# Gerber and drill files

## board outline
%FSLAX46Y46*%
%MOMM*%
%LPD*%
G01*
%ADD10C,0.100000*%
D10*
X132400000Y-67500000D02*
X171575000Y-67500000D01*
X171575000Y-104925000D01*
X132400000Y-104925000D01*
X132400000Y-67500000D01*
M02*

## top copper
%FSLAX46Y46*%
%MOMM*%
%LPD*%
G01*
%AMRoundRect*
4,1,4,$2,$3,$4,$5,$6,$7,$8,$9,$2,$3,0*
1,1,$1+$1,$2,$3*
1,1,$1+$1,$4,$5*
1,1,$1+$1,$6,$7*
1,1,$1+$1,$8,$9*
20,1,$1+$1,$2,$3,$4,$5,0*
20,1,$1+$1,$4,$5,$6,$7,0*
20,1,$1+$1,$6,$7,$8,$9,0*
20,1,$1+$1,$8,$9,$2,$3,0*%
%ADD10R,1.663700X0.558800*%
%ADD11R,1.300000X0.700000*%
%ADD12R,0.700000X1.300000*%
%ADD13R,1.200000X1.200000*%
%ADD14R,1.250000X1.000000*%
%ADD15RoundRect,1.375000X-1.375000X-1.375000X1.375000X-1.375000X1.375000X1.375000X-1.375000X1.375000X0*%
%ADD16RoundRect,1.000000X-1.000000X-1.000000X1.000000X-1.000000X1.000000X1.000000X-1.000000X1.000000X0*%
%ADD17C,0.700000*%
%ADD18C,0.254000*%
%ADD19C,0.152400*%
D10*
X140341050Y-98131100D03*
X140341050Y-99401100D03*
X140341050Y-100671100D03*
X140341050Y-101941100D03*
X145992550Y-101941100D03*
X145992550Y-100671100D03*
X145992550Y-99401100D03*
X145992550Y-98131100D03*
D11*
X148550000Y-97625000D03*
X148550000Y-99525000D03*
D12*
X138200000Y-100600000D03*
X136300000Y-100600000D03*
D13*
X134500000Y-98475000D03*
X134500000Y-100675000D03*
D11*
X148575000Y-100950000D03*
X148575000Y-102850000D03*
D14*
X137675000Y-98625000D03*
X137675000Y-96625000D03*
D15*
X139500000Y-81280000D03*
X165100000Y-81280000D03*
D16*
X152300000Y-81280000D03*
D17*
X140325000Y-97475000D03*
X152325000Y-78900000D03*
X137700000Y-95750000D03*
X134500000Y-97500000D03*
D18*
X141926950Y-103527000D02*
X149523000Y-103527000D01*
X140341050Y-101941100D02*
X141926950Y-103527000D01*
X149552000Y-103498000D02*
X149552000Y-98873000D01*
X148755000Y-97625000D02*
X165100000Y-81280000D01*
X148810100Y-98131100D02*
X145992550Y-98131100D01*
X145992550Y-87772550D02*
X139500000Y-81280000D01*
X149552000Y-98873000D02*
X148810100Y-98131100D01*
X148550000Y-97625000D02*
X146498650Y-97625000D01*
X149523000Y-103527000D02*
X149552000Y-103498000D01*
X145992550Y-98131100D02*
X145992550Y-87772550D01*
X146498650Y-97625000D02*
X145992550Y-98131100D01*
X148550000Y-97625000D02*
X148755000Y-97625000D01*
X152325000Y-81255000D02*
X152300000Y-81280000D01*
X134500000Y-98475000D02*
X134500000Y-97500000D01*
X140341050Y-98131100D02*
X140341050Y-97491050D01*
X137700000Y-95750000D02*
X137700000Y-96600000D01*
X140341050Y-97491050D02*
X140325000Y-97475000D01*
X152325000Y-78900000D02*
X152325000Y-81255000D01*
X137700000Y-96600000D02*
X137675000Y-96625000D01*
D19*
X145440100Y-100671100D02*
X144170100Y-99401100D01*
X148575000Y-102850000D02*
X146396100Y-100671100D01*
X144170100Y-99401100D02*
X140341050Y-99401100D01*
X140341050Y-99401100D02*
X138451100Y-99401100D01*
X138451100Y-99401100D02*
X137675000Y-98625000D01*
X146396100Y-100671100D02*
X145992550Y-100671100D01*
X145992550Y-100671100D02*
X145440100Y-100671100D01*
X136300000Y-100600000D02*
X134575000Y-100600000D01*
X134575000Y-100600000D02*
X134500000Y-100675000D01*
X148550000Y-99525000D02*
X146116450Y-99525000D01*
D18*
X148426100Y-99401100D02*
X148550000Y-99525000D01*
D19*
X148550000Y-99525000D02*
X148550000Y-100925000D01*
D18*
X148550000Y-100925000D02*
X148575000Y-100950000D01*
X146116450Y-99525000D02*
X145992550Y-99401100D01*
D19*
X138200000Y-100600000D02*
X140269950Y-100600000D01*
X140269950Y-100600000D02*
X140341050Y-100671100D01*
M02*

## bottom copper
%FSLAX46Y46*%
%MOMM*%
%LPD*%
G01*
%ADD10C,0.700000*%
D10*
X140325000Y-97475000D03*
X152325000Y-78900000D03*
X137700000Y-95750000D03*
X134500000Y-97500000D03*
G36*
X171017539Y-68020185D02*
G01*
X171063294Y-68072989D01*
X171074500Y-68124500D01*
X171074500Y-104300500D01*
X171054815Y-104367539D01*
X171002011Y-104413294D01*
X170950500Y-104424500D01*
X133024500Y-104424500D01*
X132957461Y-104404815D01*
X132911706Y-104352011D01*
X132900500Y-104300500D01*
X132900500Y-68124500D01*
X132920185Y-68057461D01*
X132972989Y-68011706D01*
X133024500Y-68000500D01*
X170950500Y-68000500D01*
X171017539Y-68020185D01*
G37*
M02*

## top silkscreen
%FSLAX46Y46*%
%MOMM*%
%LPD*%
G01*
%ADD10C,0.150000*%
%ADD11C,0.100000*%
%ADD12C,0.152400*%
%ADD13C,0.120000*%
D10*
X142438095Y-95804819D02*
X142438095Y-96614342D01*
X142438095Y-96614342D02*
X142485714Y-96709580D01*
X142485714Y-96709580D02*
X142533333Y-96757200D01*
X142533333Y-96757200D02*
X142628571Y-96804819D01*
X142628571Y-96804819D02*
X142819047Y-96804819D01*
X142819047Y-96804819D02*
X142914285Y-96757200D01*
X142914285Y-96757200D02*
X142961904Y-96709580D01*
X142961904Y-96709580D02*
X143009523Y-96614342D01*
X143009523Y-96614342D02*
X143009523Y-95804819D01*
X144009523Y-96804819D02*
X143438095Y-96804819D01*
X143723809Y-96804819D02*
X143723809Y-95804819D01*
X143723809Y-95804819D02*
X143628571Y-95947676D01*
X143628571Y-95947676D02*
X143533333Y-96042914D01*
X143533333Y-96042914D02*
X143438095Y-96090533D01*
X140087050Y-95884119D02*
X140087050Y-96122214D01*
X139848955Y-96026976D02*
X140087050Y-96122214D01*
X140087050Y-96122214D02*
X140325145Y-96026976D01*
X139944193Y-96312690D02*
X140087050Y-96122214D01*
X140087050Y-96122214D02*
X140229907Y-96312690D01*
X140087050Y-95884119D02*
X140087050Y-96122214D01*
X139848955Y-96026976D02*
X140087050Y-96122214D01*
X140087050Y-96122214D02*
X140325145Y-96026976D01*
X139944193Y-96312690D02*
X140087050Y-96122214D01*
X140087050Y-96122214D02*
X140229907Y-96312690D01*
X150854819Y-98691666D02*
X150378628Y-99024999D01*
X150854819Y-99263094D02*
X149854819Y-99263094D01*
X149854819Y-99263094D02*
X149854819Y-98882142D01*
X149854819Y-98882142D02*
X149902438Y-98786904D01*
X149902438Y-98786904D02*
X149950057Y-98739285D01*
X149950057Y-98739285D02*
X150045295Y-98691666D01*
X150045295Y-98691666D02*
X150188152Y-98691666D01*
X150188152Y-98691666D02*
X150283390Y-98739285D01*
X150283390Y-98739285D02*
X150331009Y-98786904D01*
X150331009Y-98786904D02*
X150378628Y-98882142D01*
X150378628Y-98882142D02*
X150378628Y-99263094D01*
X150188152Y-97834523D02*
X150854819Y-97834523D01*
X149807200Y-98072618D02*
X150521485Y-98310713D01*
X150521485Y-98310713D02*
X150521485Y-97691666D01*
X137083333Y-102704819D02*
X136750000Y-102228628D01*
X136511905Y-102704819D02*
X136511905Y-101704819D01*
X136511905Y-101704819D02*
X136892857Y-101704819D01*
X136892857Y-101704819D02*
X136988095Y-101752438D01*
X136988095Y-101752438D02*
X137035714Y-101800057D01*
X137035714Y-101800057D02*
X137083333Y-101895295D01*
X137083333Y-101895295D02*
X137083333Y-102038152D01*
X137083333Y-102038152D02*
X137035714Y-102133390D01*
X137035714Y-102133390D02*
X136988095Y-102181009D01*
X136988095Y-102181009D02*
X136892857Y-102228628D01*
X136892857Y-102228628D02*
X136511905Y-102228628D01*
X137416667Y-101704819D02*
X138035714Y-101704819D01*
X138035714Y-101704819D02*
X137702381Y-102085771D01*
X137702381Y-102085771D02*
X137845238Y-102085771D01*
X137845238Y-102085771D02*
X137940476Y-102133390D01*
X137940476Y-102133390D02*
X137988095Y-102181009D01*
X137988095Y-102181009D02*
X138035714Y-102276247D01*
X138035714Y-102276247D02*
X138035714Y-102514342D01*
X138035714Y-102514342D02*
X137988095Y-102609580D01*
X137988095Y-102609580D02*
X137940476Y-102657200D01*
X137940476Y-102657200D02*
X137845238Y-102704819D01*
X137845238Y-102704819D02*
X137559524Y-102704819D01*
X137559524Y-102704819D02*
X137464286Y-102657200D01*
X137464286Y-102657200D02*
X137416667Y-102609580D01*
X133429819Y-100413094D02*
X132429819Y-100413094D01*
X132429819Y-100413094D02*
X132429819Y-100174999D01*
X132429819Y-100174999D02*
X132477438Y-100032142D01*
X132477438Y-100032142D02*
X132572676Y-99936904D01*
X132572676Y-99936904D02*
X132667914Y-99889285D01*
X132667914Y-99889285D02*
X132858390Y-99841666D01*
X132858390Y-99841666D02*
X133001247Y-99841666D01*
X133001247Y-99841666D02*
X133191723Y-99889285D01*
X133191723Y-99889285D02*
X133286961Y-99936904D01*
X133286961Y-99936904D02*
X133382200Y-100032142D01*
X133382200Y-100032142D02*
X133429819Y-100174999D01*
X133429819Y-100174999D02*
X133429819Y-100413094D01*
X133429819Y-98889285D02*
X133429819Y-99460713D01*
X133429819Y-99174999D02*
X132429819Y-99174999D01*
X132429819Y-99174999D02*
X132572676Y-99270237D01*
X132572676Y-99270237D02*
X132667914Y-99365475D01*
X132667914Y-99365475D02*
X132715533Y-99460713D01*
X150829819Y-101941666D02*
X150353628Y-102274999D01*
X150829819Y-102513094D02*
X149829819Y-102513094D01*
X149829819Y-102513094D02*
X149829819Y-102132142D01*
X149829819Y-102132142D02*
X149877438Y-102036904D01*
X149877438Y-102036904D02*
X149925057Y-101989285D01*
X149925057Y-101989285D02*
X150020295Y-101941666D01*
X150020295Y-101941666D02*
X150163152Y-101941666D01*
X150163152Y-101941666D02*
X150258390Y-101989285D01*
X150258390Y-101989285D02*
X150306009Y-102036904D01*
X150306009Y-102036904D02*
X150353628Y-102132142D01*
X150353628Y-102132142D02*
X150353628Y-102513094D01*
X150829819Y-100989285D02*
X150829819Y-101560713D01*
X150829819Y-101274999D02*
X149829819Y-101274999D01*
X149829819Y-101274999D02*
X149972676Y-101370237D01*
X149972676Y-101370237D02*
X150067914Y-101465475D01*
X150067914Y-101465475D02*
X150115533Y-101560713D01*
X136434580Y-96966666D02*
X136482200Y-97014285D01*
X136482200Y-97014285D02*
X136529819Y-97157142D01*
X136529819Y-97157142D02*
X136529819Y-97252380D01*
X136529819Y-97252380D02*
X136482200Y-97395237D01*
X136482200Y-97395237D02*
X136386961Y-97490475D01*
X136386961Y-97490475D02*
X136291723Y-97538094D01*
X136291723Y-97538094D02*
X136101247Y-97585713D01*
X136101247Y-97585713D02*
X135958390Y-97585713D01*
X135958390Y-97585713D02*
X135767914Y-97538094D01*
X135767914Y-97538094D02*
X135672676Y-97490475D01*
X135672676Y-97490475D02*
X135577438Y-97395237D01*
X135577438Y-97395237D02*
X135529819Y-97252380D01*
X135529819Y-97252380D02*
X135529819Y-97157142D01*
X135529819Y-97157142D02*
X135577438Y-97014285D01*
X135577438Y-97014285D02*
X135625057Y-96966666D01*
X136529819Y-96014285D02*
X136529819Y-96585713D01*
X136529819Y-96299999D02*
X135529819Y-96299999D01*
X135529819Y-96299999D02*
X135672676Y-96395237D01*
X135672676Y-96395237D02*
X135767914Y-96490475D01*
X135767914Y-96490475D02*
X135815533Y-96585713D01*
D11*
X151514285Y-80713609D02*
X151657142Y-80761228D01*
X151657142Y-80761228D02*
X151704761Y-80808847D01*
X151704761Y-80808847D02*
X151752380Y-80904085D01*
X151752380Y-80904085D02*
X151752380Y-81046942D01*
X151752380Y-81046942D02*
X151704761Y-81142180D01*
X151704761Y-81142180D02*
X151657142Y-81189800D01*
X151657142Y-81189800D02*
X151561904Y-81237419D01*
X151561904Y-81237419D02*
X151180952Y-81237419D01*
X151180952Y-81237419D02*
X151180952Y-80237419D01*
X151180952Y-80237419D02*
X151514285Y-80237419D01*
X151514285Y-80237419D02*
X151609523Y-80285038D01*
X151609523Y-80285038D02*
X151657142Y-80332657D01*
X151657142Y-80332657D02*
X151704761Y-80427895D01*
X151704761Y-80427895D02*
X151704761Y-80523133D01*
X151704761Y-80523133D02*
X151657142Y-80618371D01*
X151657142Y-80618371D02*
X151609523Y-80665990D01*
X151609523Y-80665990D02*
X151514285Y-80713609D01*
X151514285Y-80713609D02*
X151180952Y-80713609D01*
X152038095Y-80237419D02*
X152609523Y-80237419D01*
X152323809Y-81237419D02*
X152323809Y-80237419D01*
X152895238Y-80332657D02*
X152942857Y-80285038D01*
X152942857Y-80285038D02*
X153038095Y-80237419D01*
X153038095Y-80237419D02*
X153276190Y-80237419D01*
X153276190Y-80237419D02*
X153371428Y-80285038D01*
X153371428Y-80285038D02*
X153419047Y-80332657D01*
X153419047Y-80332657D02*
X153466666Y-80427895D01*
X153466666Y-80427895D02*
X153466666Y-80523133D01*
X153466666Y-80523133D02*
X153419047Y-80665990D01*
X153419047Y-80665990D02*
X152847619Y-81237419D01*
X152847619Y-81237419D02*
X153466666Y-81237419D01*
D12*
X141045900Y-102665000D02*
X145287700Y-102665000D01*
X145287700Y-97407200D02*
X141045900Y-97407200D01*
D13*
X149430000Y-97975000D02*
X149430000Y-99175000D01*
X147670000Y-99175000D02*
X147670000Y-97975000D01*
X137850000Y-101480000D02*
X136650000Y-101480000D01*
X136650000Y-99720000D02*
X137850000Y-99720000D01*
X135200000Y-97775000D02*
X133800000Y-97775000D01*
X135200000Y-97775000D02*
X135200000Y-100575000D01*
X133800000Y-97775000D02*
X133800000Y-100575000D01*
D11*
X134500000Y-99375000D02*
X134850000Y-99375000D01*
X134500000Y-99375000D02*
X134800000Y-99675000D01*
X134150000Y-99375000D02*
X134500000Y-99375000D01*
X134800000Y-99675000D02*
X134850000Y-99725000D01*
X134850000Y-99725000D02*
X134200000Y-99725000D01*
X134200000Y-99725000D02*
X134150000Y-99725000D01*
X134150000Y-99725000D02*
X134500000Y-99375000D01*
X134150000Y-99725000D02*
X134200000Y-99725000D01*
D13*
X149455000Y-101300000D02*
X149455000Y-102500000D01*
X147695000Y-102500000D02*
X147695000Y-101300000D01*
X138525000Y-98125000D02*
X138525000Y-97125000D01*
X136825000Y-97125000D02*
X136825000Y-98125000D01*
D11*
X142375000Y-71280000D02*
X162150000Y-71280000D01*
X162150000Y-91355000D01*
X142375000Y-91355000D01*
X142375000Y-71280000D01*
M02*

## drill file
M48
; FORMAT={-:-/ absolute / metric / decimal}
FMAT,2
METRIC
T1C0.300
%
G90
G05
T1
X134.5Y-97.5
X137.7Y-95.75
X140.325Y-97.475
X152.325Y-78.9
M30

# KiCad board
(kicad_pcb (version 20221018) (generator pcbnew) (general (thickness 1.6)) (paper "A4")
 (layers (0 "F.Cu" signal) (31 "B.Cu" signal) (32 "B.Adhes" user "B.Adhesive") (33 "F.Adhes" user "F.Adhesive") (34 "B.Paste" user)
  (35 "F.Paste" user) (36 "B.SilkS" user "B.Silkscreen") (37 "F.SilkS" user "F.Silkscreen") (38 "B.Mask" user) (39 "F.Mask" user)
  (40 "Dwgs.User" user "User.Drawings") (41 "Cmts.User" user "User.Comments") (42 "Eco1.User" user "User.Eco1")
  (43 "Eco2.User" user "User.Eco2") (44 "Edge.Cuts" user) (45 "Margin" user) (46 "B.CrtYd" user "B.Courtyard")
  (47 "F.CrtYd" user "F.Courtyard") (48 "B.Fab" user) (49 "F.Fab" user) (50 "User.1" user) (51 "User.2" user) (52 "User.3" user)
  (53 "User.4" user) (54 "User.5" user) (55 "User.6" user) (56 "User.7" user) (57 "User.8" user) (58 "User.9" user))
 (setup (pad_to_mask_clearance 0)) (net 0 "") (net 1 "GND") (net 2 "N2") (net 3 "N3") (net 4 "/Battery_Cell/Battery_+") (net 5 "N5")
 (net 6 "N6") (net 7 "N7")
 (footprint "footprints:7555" (layer "F.Cu") (at 143.1668 100.0361)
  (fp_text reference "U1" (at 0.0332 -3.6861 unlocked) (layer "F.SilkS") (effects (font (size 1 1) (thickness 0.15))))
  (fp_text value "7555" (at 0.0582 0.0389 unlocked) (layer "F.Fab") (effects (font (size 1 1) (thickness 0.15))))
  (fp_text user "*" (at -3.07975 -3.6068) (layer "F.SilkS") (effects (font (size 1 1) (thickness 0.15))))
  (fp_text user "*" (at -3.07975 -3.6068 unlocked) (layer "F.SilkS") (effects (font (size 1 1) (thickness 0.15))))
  (fp_line (start -2.1209 2.6289) (end 2.1209 2.6289) (stroke (width 0.1524) (type solid)) (layer "F.SilkS"))
  (fp_line (start 2.1209 -2.6289) (end -2.1209 -2.6289) (stroke (width 0.1524) (type solid)) (layer "F.SilkS"))
  (pad "1" smd rect (at -2.82575 -1.905) (size 1.6637 0.5588) (layers "F.Cu" "F.Paste" "F.Mask") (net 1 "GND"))
  (pad "2" smd rect (at -2.82575 -0.635) (size 1.6637 0.5588) (layers "F.Cu" "F.Paste" "F.Mask") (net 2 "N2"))
  (pad "3" smd rect (at -2.82575 0.635) (size 1.6637 0.5588) (layers "F.Cu" "F.Paste" "F.Mask") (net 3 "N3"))
  (pad "4" smd rect (at -2.82575 1.905) (size 1.6637 0.5588) (layers "F.Cu" "F.Paste" "F.Mask") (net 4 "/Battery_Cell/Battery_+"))
  (pad "5" smd rect (at 2.82575 1.905) (size 1.6637 0.5588) (layers "F.Cu" "F.Paste" "F.Mask") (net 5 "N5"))
  (pad "6" smd rect (at 2.82575 0.635) (size 1.6637 0.5588) (layers "F.Cu" "F.Paste" "F.Mask") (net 2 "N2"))
  (pad "7" smd rect (at 2.82575 -0.635) (size 1.6637 0.5588) (layers "F.Cu" "F.Paste" "F.Mask") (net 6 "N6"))
  (pad "8" smd rect (at 2.82575 -1.905) (size 1.6637 0.5588) (layers "F.Cu" "F.Paste" "F.Mask") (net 4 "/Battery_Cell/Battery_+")))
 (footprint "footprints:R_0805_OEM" (layer "F.Cu") (at 148.55 98.575 -90)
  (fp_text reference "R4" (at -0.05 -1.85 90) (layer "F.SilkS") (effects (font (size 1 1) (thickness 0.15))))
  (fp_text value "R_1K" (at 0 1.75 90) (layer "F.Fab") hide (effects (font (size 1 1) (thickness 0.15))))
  (fp_line (start -0.6 -0.88) (end 0.6 -0.88) (stroke (width 0.12) (type solid)) (layer "F.SilkS"))
  (fp_line (start 0.6 0.88) (end -0.6 0.88) (stroke (width 0.12) (type solid)) (layer "F.SilkS"))
  (pad "1" smd rect (at -0.95 0 270) (size 0.7 1.3) (layers "F.Cu" "F.Paste" "F.Mask") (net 4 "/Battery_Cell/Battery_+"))
  (pad "2" smd rect (at 0.95 0 270) (size 0.7 1.3) (layers "F.Cu" "F.Paste" "F.Mask") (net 6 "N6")))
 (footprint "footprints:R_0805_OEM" (layer "F.Cu") (at 137.25 100.6 180)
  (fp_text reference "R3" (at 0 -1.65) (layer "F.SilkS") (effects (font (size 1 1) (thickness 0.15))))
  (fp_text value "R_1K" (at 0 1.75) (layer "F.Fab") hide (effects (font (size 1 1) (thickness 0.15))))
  (fp_line (start -0.6 -0.88) (end 0.6 -0.88) (stroke (width 0.12) (type solid)) (layer "F.SilkS"))
  (fp_line (start 0.6 0.88) (end -0.6 0.88) (stroke (width 0.12) (type solid)) (layer "F.SilkS"))
  (pad "1" smd rect (at -0.95 0 180) (size 0.7 1.3) (layers "F.Cu" "F.Paste" "F.Mask") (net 3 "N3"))
  (pad "2" smd rect (at 0.95 0 180) (size 0.7 1.3) (layers "F.Cu" "F.Paste" "F.Mask") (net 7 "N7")))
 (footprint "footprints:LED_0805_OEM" (layer "F.Cu") (at 134.5 99.575 -90)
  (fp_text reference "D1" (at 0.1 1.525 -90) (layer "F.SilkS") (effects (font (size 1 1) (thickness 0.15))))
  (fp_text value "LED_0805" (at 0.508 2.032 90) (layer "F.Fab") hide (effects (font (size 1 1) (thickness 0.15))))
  (fp_line (start -1.8 -0.7) (end -1.8 0.7) (stroke (width 0.12) (type solid)) (layer "F.SilkS"))
  (fp_line (start -1.8 -0.7) (end 1 -0.7) (stroke (width 0.12) (type solid)) (layer "F.SilkS"))
  (fp_line (start -1.8 0.7) (end 1 0.7) (stroke (width 0.12) (type solid)) (layer "F.SilkS"))
  (fp_line (start -0.2 0) (end -0.2 -0.35) (stroke (width 0.1) (type solid)) (layer "F.SilkS"))
  (fp_line (start -0.2 0) (end 0.1 -0.3) (stroke (width 0.1) (type solid)) (layer "F.SilkS"))
  (fp_line (start -0.2 0.35) (end -0.2 0) (stroke (width 0.1) (type solid)) (layer "F.SilkS"))
  (fp_line (start 0.1 -0.3) (end 0.15 -0.35) (stroke (width 0.1) (type solid)) (layer "F.SilkS"))
  (fp_line (start 0.15 -0.35) (end 0.15 0.3) (stroke (width 0.1) (type solid)) (layer "F.SilkS"))
  (fp_line (start 0.15 0.3) (end 0.15 0.35) (stroke (width 0.1) (type solid)) (layer "F.SilkS"))
  (fp_line (start 0.15 0.35) (end -0.2 0) (stroke (width 0.1) (type solid)) (layer "F.SilkS"))
  (fp_line (start 0.15 0.35) (end 0.15 0.3) (stroke (width 0.1) (type solid)) (layer "F.SilkS"))
  (pad "1" smd rect (at -1.1 0 90) (size 1.2 1.2) (layers "F.Cu" "F.Paste" "F.Mask") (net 1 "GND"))
  (pad "2" smd rect (at 1.1 0 90) (size 1.2 1.2) (layers "F.Cu" "F.Paste" "F.Mask") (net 7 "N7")))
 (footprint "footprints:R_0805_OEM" (layer "F.Cu") (at 148.575 101.9 -90)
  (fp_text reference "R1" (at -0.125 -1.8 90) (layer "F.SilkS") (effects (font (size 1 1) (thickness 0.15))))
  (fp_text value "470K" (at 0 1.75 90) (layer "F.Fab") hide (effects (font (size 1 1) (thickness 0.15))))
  (fp_line (start -0.6 -0.88) (end 0.6 -0.88) (stroke (width 0.12) (type solid)) (layer "F.SilkS"))
  (fp_line (start 0.6 0.88) (end -0.6 0.88) (stroke (width 0.12) (type solid)) (layer "F.SilkS"))
  (pad "1" smd rect (at -0.95 0 270) (size 0.7 1.3) (layers "F.Cu" "F.Paste" "F.Mask") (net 6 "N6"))
  (pad "2" smd rect (at 0.95 0 270) (size 0.7 1.3) (layers "F.Cu" "F.Paste" "F.Mask") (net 2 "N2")))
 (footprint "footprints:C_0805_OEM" (layer "F.Cu") (at 137.675 97.625 90)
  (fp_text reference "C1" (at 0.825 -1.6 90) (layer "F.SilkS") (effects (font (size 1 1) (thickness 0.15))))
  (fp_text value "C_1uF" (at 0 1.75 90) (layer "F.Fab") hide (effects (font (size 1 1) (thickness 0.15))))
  (fp_line (start -0.5 0.85) (end 0.5 0.85) (stroke (width 0.12) (type solid)) (layer "F.SilkS"))
  (fp_line (start 0.5 -0.85) (end -0.5 -0.85) (stroke (width 0.12) (type solid)) (layer "F.SilkS"))
  (pad "1" smd rect (at -1 0 90) (size 1 1.25) (layers "F.Cu" "F.Paste" "F.Mask") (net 2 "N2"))
  (pad "2" smd rect (at 1 0 90) (size 1 1.25) (layers "F.Cu" "F.Paste" "F.Mask") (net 1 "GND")))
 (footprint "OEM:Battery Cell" (layer "F.Cu") (at 152.3 81.28)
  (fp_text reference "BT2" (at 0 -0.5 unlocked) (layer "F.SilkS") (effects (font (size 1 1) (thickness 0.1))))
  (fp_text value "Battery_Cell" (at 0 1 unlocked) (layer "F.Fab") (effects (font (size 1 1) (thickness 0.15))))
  (fp_rect (start -9.925 -10) (end 9.85 10.075) (stroke (width 0.1) (type default)) (fill none) (layer "F.SilkS"))
  (pad "1" smd roundrect (at -12.8 0) (size 5.5 5.5) (layers "F.Cu" "F.Paste" "F.Mask") (roundrect_rratio 0.25)
   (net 4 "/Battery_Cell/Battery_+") (thermal_bridge_angle 45))
  (pad "2" smd roundrect (at 12.8 0) (size 5.5 5.5) (layers "F.Cu" "F.Paste" "F.Mask") (roundrect_rratio 0.25)
   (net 4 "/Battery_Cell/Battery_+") (thermal_bridge_angle 45))
  (pad "3" smd roundrect (at 0 0) (size 4 4) (layers "F.Cu" "F.Paste" "F.Mask") (roundrect_rratio 0.25) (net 1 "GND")
   (thermal_bridge_angle 45)))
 (gr_rect (start 132.4 67.5) (end 171.575 104.925) (stroke (width 0.1) (type default)) (fill none) (layer "Edge.Cuts"))
 (segment (start 141.92695 103.527) (end 149.523 103.527) (width 0.254) (layer "F.Cu") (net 4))
 (segment (start 140.34105 101.9411) (end 141.92695 103.527) (width 0.254) (layer "F.Cu") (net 4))
 (segment (start 149.552 103.498) (end 149.552 98.873) (width 0.254) (layer "F.Cu") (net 4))
 (segment (start 148.755 97.625) (end 165.1 81.28) (width 0.254) (layer "F.Cu") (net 4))
 (segment (start 148.8101 98.1311) (end 145.99255 98.1311) (width 0.254) (layer "F.Cu") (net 4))
 (segment (start 145.99255 87.77255) (end 139.5 81.28) (width 0.254) (layer "F.Cu") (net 4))
 (segment (start 149.552 98.873) (end 148.8101 98.1311) (width 0.254) (layer "F.Cu") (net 4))
 (segment (start 148.55 97.625) (end 146.49865 97.625) (width 0.254) (layer "F.Cu") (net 4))
 (segment (start 149.523 103.527) (end 149.552 103.498) (width 0.254) (layer "F.Cu") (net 4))
 (segment (start 145.99255 98.1311) (end 145.99255 87.77255) (width 0.254) (layer "F.Cu") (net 4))
 (segment (start 146.49865 97.625) (end 145.99255 98.1311) (width 0.254) (layer "F.Cu") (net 4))
 (segment (start 148.55 97.625) (end 148.755 97.625) (width 0.254) (layer "F.Cu") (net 4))
 (segment (start 152.325 81.255) (end 152.3 81.28) (width 0.254) (layer "F.Cu") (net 1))
 (segment (start 134.5 98.475) (end 134.5 97.5) (width 0.254) (layer "F.Cu") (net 1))
 (segment (start 140.34105 98.1311) (end 140.34105 97.49105) (width 0.254) (layer "F.Cu") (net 1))
 (segment (start 137.7 95.75) (end 137.7 96.6) (width 0.254) (layer "F.Cu") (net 1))
 (segment (start 140.34105 97.49105) (end 140.325 97.475) (width 0.254) (layer "F.Cu") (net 1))
 (segment (start 152.325 78.9) (end 152.325 81.255) (width 0.254) (layer "F.Cu") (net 1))
 (segment (start 137.7 96.6) (end 137.675 96.625) (width 0.254) (layer "F.Cu") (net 1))
 (via (at 140.325 97.475) (size 0.7) (drill 0.3) (layers "F.Cu" "B.Cu") (free) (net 1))
 (via (at 152.325 78.9) (size 0.7) (drill 0.3) (layers "F.Cu" "B.Cu") (free) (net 1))
 (via (at 137.7 95.75) (size 0.7) (drill 0.3) (layers "F.Cu" "B.Cu") (free) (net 1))
 (via (at 134.5 97.5) (size 0.7) (drill 0.3) (layers "F.Cu" "B.Cu") (free) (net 1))
 (segment (start 145.4401 100.6711) (end 144.1701 99.4011) (width 0.1524) (layer "F.Cu") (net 2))
 (segment (start 148.575 102.85) (end 146.3961 100.6711) (width 0.1524) (layer "F.Cu") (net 2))
 (segment (start 144.1701 99.4011) (end 140.34105 99.4011) (width 0.1524) (layer "F.Cu") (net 2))
 (segment (start 140.34105 99.4011) (end 138.4511 99.4011) (width 0.1524) (layer "F.Cu") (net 2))
 (segment (start 138.4511 99.4011) (end 137.675 98.625) (width 0.1524) (layer "F.Cu") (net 2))
 (segment (start 146.3961 100.6711) (end 145.99255 100.6711) (width 0.1524) (layer "F.Cu") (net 2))
 (segment (start 145.99255 100.6711) (end 145.4401 100.6711) (width 0.1524) (layer "F.Cu") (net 2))
 (segment (start 136.3 100.6) (end 134.575 100.6) (width 0.1524) (layer "F.Cu") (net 7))
 (segment (start 134.575 100.6) (end 134.5 100.675) (width 0.1524) (layer "F.Cu") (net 7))
 (segment (start 148.55 99.525) (end 146.11645 99.525) (width 0.1524) (layer "F.Cu") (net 6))
 (segment (start 148.4261 99.4011) (end 148.55 99.525) (width 0.254) (layer "F.Cu") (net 6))
 (segment (start 148.55 99.525) (end 148.55 100.925) (width 0.1524) (layer "F.Cu") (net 6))
 (segment (start 148.55 100.925) (end 148.575 100.95) (width 0.254) (layer "F.Cu") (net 6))
 (segment (start 146.11645 99.525) (end 145.99255 99.4011) (width 0.254) (layer "F.Cu") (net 6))
 (segment (start 138.2 100.6) (end 140.26995 100.6) (width 0.1524) (layer "F.Cu") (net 3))
 (segment (start 140.26995 100.6) (end 140.34105 100.6711) (width 0.1524) (layer "F.Cu") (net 3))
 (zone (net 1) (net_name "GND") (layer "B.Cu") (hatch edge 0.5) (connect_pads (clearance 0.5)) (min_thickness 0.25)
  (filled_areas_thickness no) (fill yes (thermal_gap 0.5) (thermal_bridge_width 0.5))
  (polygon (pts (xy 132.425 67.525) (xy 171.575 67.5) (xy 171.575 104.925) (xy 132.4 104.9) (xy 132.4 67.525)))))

